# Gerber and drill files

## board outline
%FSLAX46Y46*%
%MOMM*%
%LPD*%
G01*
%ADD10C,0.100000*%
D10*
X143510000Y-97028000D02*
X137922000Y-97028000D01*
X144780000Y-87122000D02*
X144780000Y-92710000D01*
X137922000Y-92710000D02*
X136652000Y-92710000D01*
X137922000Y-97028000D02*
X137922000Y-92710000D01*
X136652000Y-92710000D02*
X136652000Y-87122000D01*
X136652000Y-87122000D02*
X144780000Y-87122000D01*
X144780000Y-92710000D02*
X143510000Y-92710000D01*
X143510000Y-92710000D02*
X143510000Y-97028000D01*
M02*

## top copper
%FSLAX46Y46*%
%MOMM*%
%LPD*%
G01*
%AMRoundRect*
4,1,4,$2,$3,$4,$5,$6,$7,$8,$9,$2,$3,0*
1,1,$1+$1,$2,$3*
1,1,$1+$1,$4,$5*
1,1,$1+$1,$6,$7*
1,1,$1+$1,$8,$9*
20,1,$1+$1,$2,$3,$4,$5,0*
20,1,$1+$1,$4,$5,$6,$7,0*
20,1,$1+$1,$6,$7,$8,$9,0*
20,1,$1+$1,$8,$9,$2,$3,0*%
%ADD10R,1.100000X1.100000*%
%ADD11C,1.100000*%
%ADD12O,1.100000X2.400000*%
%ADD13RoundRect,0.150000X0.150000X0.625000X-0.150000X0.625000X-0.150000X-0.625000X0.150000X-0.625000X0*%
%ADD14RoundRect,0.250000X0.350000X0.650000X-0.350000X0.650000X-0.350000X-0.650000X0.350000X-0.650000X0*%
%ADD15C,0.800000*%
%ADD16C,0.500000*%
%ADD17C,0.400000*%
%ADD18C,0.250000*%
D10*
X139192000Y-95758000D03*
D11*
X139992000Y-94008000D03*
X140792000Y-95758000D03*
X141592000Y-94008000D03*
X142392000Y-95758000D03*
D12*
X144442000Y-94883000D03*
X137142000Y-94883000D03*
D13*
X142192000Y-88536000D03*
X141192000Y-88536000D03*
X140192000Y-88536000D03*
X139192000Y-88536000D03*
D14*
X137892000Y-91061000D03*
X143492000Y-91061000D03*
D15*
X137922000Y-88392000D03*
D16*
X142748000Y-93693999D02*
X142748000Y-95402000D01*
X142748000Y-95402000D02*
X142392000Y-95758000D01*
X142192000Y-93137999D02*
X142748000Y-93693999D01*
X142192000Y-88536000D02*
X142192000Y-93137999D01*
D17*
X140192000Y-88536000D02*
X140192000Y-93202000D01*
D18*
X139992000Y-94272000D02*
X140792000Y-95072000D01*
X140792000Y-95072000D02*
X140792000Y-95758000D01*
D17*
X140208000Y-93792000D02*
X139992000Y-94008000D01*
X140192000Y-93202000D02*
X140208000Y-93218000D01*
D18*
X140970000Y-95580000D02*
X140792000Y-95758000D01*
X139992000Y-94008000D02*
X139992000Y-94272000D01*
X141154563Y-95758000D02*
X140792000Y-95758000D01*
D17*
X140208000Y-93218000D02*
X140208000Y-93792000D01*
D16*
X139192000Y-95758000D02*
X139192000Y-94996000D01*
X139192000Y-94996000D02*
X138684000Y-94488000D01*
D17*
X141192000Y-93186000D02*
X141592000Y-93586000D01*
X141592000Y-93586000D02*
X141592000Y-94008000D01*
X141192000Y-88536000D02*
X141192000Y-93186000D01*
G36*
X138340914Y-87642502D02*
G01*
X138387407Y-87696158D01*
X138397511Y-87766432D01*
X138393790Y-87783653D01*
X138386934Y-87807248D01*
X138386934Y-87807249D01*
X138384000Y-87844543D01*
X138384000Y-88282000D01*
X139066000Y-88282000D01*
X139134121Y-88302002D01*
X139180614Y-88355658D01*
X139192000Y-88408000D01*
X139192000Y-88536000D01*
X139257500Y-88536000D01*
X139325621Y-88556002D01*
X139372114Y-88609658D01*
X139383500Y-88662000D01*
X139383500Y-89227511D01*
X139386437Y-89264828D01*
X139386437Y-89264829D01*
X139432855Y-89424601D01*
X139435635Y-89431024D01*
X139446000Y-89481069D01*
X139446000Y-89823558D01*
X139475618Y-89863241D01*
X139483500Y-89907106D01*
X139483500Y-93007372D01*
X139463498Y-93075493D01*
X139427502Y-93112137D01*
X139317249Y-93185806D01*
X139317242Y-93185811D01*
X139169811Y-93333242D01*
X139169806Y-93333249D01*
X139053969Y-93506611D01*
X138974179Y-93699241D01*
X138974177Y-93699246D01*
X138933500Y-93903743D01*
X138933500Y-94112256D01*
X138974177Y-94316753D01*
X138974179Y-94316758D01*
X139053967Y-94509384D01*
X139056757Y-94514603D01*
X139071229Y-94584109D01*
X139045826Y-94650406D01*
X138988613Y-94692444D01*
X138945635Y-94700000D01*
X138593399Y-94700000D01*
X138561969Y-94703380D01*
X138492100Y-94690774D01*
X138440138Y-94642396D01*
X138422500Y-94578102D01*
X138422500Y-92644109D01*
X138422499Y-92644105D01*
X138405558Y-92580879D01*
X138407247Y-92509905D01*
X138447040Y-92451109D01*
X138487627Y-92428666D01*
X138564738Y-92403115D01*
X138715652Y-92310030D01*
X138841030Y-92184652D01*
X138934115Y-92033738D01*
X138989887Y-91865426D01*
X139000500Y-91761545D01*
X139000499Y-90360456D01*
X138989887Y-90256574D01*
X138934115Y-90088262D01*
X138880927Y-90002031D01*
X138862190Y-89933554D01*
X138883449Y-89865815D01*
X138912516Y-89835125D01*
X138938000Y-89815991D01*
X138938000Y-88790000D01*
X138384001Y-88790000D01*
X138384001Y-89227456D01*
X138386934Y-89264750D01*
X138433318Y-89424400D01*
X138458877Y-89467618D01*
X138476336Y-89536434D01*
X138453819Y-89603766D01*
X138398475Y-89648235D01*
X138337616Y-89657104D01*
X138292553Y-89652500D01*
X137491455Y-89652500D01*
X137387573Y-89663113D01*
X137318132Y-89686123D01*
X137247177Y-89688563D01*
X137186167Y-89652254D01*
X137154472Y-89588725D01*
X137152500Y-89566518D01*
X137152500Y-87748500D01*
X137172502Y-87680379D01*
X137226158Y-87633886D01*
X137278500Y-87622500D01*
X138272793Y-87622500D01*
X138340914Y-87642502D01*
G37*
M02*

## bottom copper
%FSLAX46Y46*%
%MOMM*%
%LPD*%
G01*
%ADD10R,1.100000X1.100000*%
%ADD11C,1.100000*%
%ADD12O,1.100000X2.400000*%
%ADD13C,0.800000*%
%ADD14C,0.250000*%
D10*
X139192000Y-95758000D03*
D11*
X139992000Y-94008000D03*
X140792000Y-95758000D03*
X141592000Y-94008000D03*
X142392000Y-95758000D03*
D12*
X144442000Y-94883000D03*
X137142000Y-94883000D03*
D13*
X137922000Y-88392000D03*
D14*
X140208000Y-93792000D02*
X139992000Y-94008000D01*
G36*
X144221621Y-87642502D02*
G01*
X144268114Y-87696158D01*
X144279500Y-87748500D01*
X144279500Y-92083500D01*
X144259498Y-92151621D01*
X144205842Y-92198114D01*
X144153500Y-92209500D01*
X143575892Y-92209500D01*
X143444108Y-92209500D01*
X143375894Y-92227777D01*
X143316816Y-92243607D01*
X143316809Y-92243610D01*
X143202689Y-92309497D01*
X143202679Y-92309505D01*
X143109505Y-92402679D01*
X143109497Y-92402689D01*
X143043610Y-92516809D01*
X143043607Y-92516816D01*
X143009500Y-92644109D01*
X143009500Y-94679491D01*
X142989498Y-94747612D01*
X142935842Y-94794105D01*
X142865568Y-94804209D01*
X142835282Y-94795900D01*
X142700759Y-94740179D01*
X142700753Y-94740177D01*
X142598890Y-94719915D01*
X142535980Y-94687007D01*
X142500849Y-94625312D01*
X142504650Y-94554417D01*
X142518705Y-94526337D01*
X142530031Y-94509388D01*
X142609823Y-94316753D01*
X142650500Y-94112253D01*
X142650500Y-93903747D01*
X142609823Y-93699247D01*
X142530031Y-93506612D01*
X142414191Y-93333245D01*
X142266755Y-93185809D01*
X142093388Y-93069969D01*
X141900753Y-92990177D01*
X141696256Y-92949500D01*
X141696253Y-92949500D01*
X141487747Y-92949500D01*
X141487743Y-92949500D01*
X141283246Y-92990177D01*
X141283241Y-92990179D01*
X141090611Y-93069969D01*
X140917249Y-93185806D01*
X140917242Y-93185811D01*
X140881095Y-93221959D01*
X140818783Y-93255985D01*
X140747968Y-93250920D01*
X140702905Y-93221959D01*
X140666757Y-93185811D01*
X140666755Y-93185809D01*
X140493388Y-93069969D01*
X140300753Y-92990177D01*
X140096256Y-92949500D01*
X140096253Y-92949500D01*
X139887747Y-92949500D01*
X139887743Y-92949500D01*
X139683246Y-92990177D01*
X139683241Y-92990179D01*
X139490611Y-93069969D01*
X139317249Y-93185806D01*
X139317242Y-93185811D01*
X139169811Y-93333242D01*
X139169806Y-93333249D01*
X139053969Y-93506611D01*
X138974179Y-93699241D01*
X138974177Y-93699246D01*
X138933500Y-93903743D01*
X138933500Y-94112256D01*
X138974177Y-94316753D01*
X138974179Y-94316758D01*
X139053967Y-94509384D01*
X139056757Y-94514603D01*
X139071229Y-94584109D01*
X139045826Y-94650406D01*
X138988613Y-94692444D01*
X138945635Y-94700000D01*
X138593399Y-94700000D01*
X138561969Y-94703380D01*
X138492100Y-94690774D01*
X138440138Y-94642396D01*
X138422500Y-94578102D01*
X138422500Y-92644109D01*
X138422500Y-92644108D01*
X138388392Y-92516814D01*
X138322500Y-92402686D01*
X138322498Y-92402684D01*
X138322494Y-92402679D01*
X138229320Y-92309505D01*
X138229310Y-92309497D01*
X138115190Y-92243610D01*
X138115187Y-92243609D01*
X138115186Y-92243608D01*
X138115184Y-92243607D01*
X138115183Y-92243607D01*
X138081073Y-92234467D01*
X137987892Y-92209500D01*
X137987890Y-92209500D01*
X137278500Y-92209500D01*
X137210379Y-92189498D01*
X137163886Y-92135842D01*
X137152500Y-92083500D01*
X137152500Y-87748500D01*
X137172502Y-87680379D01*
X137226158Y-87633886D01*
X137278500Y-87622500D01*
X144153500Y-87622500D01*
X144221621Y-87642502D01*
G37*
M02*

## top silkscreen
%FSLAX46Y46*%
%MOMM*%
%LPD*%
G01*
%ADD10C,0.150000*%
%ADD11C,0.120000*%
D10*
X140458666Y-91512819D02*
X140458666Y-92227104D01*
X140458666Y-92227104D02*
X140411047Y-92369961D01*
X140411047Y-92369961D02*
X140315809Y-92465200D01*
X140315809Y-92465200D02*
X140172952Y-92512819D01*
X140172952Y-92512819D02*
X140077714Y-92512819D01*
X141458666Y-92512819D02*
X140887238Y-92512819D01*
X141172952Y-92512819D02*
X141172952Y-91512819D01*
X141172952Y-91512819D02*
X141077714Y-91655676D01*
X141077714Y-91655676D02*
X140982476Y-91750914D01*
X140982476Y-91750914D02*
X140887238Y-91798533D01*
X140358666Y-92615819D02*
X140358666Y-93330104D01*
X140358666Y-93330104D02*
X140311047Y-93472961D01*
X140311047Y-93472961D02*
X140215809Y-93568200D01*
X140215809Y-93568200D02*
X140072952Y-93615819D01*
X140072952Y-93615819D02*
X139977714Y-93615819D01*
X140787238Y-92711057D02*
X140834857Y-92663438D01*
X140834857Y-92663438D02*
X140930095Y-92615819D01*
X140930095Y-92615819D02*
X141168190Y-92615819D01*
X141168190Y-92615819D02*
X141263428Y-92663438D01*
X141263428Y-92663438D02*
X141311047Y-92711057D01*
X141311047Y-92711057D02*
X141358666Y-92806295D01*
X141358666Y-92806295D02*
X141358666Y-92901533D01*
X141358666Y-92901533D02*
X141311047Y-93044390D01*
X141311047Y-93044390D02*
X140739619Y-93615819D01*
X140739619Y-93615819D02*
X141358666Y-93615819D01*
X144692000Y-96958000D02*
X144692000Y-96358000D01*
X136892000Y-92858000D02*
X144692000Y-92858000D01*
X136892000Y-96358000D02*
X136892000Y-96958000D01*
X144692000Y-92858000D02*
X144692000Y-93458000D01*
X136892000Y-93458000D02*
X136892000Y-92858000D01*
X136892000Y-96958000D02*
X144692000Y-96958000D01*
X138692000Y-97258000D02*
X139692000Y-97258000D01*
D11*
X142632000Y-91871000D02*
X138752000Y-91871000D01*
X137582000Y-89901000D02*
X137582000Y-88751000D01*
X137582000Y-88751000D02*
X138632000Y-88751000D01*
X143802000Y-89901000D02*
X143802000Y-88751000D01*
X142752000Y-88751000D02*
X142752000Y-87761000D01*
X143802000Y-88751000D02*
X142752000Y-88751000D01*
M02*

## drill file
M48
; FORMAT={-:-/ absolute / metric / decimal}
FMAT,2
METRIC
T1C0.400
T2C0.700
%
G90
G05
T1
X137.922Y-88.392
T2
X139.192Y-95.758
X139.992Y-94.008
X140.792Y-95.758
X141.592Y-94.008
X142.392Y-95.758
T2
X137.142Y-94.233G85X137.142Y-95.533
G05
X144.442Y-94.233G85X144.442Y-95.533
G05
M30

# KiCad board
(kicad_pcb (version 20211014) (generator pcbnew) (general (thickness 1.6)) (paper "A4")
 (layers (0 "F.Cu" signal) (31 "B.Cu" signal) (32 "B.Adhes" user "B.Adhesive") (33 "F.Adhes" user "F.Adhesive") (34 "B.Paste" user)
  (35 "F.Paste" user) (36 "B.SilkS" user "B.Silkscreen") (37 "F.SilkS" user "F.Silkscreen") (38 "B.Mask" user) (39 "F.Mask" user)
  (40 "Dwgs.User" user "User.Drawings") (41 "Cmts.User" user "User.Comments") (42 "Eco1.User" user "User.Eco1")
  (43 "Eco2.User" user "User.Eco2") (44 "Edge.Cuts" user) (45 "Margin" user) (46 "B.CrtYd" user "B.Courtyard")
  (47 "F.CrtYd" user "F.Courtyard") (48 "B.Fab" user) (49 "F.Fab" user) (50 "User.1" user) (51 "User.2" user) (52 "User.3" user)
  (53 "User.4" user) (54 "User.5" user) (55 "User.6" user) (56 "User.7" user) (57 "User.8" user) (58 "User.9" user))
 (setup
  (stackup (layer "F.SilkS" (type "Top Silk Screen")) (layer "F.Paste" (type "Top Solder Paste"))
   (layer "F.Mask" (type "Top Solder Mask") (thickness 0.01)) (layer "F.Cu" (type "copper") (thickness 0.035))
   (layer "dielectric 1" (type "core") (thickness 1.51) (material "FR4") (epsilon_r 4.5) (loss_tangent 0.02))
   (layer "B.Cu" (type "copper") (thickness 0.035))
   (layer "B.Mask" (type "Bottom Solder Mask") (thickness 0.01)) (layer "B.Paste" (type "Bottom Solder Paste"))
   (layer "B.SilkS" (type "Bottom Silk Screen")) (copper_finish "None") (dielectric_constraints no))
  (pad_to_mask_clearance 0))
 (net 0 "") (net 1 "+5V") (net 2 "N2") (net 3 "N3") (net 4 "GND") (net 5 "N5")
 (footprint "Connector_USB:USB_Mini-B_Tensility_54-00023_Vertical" (layer "F.Cu") (at 139.192 95.758)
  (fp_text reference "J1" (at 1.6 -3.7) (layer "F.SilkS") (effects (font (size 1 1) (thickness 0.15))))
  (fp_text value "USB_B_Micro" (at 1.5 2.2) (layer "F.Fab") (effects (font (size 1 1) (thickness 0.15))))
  (fp_line (start 5.5 1.2) (end 5.5 0.6) (layer "F.SilkS") (width 0.15))
  (fp_line (start -2.3 -2.9) (end 5.5 -2.9) (layer "F.SilkS") (width 0.15))
  (fp_line (start -2.3 0.6) (end -2.3 1.2) (layer "F.SilkS") (width 0.15))
  (fp_line (start 5.5 -2.9) (end 5.5 -2.3) (layer "F.SilkS") (width 0.15))
  (fp_line (start -2.3 -2.3) (end -2.3 -2.9) (layer "F.SilkS") (width 0.15))
  (fp_line (start -2.3 1.2) (end 5.5 1.2) (layer "F.SilkS") (width 0.15))
  (fp_line (start -0.5 1.5) (end 0.5 1.5) (layer "F.SilkS") (width 0.15))
  (pad "1" thru_hole rect (at 0 0) (size 1.1 1.1) (drill 0.7) (layers *.Cu *.Mask) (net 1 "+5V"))
  (pad "2" thru_hole circle (at 0.8 -1.75) (size 1.1 1.1) (drill 0.7) (layers *.Cu *.Mask) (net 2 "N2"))
  (pad "3" thru_hole circle (at 1.6 0) (size 1.1 1.1) (drill 0.7) (layers *.Cu *.Mask) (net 2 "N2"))
  (pad "4" thru_hole circle (at 2.4 -1.75) (size 1.1 1.1) (drill 0.7) (layers *.Cu *.Mask) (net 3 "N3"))
  (pad "5" thru_hole circle (at 3.2 0) (size 1.1 1.1) (drill 0.7) (layers *.Cu *.Mask) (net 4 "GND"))
  (pad "6" thru_hole oval (at 5.25 -0.875) (size 1.1 2.4) (drill oval 0.7 2) (layers *.Cu *.Mask) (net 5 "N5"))
  (pad "6" thru_hole oval (at -2.05 -0.875) (size 1.1 2.4) (drill oval 0.7 2) (layers *.Cu *.Mask) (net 5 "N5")))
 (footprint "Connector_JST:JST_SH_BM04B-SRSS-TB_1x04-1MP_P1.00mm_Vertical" (layer "F.Cu") (at 140.692 89.861 180)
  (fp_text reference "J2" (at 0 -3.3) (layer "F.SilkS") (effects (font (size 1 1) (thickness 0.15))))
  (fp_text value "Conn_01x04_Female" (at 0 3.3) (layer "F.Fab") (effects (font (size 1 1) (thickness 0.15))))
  (fp_line (start -1.94 -2.01) (end 1.94 -2.01) (layer "F.SilkS") (width 0.12))
  (fp_line (start 3.11 -0.04) (end 3.11 1.11) (layer "F.SilkS") (width 0.12))
  (fp_line (start 3.11 1.11) (end 2.06 1.11) (layer "F.SilkS") (width 0.12))
  (fp_line (start -3.11 -0.04) (end -3.11 1.11) (layer "F.SilkS") (width 0.12))
  (fp_line (start -2.06 1.11) (end -2.06 2.1) (layer "F.SilkS") (width 0.12))
  (fp_line (start -3.11 1.11) (end -2.06 1.11) (layer "F.SilkS") (width 0.12))
  (pad "1" smd roundrect (at -1.5 1.325 180) (size 0.6 1.55) (layers "F.Cu" "F.Paste" "F.Mask") (roundrect_rratio 0.25) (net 4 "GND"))
  (pad "2" smd roundrect (at -0.5 1.325 180) (size 0.6 1.55) (layers "F.Cu" "F.Paste" "F.Mask") (roundrect_rratio 0.25) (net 3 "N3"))
  (pad "3" smd roundrect (at 0.5 1.325 180) (size 0.6 1.55) (layers "F.Cu" "F.Paste" "F.Mask") (roundrect_rratio 0.25) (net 2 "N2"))
  (pad "4" smd roundrect (at 1.5 1.325 180) (size 0.6 1.55) (layers "F.Cu" "F.Paste" "F.Mask") (roundrect_rratio 0.25) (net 1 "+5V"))
  (pad "MP" smd roundrect (at 2.8 -1.2 180) (size 1.2 1.8) (layers "F.Cu" "F.Paste" "F.Mask") (roundrect_rratio 0.208333))
  (pad "MP" smd roundrect (at -2.8 -1.2 180) (size 1.2 1.8) (layers "F.Cu" "F.Paste" "F.Mask") (roundrect_rratio 0.208333)))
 (gr_line (start 143.51 97.028) (end 137.922 97.028) (layer "Edge.Cuts") (width 0.1))
 (gr_line (start 144.78 87.122) (end 144.78 92.71) (layer "Edge.Cuts") (width 0.1))
 (gr_line (start 137.922 92.71) (end 136.652 92.71) (layer "Edge.Cuts") (width 0.1))
 (gr_line (start 137.922 97.028) (end 137.922 92.71) (layer "Edge.Cuts") (width 0.1))
 (gr_line (start 136.652 92.71) (end 136.652 87.122) (layer "Edge.Cuts") (width 0.1))
 (gr_line (start 136.652 87.122) (end 144.78 87.122) (layer "Edge.Cuts") (width 0.1))
 (gr_line (start 144.78 92.71) (end 143.51 92.71) (layer "Edge.Cuts") (width 0.1))
 (gr_line (start 143.51 92.71) (end 143.51 97.028) (layer "Edge.Cuts") (width 0.1))
 (segment (start 142.748 93.693999) (end 142.748 95.402) (width 0.5) (layer "F.Cu") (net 4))
 (segment (start 142.748 95.402) (end 142.392 95.758) (width 0.5) (layer "F.Cu") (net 4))
 (segment (start 142.192 93.137999) (end 142.748 93.693999) (width 0.5) (layer "F.Cu") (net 4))
 (segment (start 142.192 88.536) (end 142.192 93.137999) (width 0.5) (layer "F.Cu") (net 4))
 (segment (start 140.192 88.536) (end 140.192 93.202) (width 0.4) (layer "F.Cu") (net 2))
 (segment (start 139.992 94.272) (end 140.792 95.072) (width 0.25) (layer "F.Cu") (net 2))
 (segment (start 140.792 95.072) (end 140.792 95.758) (width 0.25) (layer "F.Cu") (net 2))
 (segment (start 140.208 93.792) (end 139.992 94.008) (width 0.4) (layer "F.Cu") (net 2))
 (segment (start 140.192 93.202) (end 140.208 93.218) (width 0.4) (layer "F.Cu") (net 2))
 (segment (start 140.97 95.58) (end 140.792 95.758) (width 0.25) (layer "F.Cu") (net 2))
 (segment (start 139.992 94.008) (end 139.992 94.272) (width 0.25) (layer "F.Cu") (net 2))
 (segment (start 141.154563 95.758) (end 140.792 95.758) (width 0.25) (layer "F.Cu") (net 2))
 (segment (start 140.208 93.218) (end 140.208 93.792) (width 0.4) (layer "F.Cu") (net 2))
 (segment (start 140.208 93.792) (end 139.992 94.008) (width 0.25) (layer "B.Cu") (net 2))
 (segment (start 139.192 95.758) (end 139.192 94.996) (width 0.5) (layer "F.Cu") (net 1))
 (segment (start 139.192 94.996) (end 138.684 94.488) (width 0.5) (layer "F.Cu") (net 1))
 (via (at 137.922 88.392) (size 0.8) (drill 0.4) (layers "F.Cu" "B.Cu") (free) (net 1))
 (segment (start 141.192 93.186) (end 141.592 93.586) (width 0.4) (layer "F.Cu") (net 3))
 (segment (start 141.592 93.586) (end 141.592 94.008) (width 0.4) (layer "F.Cu") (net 3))
 (segment (start 141.192 88.536) (end 141.192 93.186) (width 0.4) (layer "F.Cu") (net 3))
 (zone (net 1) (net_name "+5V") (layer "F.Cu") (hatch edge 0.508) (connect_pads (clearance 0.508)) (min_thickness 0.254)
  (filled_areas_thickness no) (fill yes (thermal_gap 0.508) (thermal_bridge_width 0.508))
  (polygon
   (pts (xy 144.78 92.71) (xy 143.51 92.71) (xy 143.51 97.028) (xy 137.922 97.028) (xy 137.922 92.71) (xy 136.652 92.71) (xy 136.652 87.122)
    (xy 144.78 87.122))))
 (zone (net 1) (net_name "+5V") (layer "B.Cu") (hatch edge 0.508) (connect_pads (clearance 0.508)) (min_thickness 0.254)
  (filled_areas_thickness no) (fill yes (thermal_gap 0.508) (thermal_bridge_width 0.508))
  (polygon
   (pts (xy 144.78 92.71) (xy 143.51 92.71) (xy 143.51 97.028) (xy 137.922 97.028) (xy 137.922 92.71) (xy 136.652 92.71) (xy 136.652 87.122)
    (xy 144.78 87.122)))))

